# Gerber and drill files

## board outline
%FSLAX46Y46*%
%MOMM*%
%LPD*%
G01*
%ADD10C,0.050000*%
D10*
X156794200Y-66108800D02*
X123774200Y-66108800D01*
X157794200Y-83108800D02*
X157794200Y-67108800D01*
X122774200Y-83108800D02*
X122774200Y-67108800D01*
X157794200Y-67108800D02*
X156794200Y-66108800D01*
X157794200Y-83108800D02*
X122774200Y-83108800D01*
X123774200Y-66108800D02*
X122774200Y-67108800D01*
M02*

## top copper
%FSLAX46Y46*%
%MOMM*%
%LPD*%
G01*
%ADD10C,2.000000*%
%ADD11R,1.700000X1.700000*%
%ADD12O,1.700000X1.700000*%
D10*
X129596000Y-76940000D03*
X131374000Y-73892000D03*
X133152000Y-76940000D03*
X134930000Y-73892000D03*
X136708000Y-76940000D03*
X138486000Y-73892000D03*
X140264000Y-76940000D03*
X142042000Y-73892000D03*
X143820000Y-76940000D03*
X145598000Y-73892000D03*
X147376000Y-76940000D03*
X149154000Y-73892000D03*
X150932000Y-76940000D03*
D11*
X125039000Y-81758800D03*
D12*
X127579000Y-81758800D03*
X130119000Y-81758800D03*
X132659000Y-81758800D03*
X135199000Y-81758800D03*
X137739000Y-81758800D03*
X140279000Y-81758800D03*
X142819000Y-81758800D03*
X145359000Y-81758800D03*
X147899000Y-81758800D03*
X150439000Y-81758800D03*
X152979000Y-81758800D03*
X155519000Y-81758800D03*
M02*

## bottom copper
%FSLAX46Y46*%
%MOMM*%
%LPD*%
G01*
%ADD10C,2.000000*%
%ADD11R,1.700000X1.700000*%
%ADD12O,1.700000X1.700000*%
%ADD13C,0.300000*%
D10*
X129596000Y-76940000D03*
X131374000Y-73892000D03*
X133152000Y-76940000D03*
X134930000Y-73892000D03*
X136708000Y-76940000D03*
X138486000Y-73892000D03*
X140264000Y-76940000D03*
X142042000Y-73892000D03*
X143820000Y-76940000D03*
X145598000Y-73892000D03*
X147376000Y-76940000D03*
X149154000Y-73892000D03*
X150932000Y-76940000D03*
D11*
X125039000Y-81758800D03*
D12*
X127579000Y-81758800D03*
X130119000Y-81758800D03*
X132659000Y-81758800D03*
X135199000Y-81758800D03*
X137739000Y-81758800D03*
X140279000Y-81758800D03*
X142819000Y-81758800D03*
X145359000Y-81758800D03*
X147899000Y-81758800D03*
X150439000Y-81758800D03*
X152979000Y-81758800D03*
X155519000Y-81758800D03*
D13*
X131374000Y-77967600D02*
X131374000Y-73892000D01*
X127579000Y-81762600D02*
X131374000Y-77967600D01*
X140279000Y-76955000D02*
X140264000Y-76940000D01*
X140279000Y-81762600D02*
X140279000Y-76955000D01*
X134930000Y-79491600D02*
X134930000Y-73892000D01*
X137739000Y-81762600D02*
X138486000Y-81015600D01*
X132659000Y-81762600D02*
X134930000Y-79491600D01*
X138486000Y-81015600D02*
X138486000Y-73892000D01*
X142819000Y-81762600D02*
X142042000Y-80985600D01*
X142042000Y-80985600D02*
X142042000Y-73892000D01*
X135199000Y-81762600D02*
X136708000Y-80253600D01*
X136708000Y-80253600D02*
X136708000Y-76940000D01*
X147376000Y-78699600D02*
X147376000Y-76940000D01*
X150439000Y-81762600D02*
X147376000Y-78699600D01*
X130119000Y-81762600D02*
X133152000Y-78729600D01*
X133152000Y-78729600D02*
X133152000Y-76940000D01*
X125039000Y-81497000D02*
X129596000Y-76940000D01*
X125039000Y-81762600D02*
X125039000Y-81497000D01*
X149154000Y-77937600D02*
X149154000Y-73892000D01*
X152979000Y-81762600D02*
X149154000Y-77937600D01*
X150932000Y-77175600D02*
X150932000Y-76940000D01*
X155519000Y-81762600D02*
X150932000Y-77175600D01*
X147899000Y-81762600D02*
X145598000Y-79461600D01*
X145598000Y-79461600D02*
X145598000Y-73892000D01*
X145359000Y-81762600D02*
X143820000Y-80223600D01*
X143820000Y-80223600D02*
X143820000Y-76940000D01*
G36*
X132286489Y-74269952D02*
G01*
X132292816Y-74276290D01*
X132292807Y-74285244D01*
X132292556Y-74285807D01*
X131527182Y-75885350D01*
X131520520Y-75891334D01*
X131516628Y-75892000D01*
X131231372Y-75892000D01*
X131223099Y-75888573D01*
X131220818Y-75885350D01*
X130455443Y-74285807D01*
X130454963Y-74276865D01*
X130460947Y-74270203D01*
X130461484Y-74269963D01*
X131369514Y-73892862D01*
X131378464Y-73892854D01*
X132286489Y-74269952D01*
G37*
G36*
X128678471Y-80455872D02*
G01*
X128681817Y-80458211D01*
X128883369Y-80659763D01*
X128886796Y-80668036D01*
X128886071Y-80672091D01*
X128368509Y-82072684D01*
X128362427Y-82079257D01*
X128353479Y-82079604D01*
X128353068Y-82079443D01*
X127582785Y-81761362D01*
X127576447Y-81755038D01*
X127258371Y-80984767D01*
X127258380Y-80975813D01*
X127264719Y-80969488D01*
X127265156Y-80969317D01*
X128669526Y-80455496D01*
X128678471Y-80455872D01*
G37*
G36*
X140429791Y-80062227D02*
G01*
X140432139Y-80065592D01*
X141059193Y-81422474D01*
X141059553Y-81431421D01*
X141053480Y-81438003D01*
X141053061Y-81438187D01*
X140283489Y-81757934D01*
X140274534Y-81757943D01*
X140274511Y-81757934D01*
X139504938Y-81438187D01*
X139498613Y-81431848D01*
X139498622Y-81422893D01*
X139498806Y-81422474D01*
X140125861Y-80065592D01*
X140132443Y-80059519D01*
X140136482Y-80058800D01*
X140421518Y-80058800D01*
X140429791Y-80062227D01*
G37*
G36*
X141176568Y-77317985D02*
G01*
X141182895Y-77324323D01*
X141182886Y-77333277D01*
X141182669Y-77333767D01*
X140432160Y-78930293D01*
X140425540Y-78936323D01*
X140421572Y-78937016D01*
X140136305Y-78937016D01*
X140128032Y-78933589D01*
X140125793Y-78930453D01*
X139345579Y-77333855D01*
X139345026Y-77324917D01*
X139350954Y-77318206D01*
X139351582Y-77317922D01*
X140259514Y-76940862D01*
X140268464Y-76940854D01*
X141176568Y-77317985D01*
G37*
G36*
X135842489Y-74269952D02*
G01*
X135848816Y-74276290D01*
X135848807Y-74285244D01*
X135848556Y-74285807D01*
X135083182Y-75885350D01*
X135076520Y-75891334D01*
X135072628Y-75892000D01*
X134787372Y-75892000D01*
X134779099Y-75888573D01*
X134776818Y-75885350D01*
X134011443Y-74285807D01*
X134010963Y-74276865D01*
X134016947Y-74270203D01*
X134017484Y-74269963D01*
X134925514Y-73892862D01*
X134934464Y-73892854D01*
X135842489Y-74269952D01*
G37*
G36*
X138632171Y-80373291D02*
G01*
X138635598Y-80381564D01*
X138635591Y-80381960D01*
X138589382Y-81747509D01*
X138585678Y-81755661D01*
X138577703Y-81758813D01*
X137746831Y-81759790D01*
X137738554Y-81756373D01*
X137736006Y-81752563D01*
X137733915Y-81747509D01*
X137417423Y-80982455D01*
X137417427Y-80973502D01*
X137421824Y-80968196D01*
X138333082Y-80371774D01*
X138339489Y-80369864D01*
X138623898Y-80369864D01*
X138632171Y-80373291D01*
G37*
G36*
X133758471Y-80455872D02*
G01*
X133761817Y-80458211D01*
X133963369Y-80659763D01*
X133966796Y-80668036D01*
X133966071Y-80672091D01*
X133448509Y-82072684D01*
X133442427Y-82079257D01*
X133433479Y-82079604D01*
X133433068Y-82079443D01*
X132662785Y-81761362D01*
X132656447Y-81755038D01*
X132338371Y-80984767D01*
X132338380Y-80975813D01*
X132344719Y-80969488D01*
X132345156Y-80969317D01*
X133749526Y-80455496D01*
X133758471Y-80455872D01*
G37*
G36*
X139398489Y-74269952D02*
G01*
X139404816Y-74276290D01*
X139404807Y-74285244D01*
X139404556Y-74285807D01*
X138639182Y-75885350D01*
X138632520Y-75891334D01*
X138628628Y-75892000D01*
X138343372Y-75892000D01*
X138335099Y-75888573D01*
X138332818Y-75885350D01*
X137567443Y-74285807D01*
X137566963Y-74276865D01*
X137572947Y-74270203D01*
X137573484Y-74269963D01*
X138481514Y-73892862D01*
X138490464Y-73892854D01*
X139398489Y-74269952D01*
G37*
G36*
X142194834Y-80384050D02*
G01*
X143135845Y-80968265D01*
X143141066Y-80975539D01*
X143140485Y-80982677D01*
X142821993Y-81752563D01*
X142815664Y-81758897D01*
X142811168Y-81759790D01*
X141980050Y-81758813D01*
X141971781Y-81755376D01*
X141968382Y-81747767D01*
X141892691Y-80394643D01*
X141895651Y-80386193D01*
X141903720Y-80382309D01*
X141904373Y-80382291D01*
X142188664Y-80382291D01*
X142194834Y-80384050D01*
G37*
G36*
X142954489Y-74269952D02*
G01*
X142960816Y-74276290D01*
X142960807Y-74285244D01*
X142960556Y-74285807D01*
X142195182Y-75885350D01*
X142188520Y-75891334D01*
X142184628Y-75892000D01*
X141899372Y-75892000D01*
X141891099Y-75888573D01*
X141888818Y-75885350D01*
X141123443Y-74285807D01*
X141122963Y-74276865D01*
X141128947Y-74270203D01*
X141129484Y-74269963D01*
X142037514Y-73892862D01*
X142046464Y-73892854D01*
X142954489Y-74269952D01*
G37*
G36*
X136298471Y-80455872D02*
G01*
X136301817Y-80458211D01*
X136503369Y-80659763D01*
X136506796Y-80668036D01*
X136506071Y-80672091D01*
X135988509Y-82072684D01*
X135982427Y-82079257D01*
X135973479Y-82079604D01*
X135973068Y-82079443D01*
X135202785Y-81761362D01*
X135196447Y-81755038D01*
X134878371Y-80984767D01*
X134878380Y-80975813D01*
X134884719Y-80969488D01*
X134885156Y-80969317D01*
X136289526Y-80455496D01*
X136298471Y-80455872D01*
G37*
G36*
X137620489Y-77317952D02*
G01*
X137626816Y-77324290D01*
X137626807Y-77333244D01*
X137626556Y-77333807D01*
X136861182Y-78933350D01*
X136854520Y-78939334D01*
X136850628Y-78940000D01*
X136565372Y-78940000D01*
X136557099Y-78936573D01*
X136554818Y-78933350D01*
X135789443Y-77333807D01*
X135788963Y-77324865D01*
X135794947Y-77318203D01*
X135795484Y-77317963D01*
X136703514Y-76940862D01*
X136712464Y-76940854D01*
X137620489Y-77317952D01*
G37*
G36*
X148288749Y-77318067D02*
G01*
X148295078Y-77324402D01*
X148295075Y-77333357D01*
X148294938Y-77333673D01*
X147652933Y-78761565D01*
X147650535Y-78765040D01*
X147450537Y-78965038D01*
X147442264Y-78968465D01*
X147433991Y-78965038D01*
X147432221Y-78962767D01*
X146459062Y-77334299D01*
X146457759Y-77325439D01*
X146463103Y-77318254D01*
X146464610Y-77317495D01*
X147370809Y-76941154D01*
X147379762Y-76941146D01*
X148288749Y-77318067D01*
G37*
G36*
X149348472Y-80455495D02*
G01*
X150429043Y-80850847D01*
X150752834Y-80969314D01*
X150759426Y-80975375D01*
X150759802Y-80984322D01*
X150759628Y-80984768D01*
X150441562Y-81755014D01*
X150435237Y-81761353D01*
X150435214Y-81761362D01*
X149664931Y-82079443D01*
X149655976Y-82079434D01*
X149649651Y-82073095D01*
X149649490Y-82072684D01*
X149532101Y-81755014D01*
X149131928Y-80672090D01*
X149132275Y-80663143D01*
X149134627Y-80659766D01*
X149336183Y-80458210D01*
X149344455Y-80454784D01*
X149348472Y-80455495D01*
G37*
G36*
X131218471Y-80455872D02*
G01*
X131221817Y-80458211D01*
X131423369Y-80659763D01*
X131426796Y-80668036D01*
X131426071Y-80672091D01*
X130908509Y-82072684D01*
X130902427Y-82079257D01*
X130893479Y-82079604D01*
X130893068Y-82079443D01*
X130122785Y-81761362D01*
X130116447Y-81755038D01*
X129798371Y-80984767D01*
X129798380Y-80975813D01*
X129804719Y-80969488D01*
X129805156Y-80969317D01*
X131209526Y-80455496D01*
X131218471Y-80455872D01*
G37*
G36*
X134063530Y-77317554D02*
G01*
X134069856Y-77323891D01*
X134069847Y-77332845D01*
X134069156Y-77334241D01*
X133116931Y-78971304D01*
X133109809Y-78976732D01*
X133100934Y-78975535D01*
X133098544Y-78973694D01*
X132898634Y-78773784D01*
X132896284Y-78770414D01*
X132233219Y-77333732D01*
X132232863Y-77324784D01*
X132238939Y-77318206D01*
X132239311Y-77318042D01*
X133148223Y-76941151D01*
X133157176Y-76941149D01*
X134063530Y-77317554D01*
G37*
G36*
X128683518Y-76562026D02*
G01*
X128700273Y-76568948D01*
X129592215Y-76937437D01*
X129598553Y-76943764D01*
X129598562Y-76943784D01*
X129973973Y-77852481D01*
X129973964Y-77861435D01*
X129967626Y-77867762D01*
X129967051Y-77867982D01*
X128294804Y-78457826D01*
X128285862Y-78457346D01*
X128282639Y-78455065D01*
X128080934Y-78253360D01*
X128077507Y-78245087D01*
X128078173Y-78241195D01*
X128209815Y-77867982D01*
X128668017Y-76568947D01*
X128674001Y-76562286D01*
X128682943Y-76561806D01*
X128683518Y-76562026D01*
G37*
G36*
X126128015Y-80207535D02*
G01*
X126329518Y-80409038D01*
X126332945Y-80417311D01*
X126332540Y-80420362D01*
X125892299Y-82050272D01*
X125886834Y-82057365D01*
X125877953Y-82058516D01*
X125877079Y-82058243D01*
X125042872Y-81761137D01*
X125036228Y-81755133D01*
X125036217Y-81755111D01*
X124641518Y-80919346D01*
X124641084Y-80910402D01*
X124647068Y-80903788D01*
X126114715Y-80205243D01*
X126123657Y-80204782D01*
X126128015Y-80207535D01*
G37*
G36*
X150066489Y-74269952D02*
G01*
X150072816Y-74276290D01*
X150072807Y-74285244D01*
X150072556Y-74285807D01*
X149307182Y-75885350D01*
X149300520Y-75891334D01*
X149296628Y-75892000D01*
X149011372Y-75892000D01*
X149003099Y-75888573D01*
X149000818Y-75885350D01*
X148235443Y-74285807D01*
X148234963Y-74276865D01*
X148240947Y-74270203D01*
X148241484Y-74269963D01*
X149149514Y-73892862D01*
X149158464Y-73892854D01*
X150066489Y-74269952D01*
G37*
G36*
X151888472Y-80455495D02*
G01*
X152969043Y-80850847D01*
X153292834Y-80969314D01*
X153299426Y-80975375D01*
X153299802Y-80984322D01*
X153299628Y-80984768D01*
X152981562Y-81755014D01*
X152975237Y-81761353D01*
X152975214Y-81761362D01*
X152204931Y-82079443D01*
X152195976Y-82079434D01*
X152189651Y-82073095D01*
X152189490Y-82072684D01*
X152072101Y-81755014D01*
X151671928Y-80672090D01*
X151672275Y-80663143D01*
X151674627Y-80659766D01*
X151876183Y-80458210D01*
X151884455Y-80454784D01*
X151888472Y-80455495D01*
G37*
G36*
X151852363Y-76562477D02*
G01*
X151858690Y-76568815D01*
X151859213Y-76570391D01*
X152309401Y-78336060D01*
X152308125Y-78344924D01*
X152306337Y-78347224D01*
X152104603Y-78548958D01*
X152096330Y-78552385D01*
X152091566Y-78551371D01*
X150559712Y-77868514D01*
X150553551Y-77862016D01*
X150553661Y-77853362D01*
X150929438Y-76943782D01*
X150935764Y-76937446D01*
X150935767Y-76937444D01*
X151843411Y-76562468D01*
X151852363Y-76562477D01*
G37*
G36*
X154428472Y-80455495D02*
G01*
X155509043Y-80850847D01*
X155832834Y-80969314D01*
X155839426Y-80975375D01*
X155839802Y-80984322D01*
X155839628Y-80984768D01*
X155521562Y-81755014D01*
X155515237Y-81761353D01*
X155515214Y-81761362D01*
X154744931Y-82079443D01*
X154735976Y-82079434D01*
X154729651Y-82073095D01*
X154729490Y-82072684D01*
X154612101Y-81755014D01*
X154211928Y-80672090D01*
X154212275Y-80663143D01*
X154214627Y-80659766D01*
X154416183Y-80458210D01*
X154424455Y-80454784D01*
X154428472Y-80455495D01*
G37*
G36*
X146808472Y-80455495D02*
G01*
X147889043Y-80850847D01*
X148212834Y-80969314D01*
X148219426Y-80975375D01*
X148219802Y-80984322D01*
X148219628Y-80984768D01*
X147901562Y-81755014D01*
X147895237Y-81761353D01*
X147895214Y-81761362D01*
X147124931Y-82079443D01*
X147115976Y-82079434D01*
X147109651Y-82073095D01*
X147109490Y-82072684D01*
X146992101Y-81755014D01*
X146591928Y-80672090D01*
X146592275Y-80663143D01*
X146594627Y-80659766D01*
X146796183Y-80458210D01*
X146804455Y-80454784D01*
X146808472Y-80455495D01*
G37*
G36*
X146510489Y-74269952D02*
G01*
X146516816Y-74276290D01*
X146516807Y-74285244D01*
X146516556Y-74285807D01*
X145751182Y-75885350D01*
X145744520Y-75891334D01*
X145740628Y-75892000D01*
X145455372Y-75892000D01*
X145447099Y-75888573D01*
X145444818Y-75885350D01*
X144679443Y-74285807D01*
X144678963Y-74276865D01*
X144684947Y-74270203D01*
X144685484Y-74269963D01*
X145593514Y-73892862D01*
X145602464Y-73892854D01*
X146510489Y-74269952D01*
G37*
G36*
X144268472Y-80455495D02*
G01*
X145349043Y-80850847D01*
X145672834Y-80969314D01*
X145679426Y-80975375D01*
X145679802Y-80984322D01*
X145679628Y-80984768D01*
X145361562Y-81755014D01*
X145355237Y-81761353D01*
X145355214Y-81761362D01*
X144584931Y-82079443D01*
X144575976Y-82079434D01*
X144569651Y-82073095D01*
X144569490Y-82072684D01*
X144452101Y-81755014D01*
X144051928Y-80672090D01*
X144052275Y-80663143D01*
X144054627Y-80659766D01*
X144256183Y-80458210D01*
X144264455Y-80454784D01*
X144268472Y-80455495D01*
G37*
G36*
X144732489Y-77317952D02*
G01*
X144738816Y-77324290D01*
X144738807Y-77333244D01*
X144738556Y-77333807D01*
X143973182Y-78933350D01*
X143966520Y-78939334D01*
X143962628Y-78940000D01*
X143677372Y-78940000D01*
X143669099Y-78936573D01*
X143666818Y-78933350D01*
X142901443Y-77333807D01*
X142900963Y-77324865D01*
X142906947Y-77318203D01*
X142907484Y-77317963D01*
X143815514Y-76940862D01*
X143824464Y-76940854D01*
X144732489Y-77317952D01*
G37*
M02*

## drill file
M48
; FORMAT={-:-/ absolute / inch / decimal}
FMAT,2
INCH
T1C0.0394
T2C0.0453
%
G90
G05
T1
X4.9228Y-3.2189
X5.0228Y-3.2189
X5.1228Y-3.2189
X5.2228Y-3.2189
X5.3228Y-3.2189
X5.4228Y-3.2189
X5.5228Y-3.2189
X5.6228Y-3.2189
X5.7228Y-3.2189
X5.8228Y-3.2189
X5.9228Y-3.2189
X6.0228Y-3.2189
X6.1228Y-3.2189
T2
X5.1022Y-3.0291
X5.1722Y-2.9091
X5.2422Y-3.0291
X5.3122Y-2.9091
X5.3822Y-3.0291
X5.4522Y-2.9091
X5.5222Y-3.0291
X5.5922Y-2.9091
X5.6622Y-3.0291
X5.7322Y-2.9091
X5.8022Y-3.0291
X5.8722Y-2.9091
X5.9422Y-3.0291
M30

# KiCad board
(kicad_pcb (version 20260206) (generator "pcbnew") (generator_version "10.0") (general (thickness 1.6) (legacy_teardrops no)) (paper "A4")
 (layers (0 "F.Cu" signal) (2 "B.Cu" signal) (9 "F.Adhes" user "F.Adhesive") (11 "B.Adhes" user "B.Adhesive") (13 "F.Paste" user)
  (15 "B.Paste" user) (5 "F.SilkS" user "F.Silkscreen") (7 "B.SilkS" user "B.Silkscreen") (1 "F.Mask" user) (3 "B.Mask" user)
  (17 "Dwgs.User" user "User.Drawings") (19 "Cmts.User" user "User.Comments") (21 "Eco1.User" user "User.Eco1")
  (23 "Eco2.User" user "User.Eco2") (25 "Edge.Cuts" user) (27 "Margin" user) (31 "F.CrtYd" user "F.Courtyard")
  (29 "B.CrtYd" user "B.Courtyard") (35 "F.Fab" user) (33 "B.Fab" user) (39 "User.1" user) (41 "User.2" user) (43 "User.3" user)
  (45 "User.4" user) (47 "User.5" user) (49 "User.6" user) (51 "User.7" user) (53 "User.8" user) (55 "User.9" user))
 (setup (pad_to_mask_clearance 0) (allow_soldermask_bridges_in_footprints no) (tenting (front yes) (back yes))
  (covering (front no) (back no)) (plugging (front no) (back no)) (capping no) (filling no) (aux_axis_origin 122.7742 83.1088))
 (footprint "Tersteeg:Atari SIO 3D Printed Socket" (layer "F.Cu") (at 129.596 83.036)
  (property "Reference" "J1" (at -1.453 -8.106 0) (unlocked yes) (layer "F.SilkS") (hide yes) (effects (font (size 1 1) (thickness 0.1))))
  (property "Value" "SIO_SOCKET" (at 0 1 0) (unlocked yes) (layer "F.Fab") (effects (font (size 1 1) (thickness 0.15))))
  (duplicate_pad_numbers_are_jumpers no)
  (pad "1" thru_hole circle (at 0 -6.096) (size 2 2) (drill 1.15) (layers "*.Cu" "*.Mask") (remove_unused_layers no)
   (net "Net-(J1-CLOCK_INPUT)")
   (teardrops (best_length_ratio 0.5) (max_length 1) (best_width_ratio 1) (max_width 2) (curved_edges no) (filter_ratio 0.9) (enabled yes)
    (allow_two_segments yes) (prefer_zone_connections yes)))
  (pad "2" thru_hole circle (at 1.778 -9.144) (size 2 2) (drill 1.15) (layers "*.Cu" "*.Mask") (remove_unused_layers no)
   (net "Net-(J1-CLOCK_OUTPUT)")
   (teardrops (best_length_ratio 0.5) (max_length 1) (best_width_ratio 1) (max_width 2) (curved_edges no) (filter_ratio 0.9) (enabled yes)
    (allow_two_segments yes) (prefer_zone_connections yes)))
  (pad "3" thru_hole circle (at 3.556 -6.096) (size 2 2) (drill 1.15) (layers "*.Cu" "*.Mask") (remove_unused_layers no)
   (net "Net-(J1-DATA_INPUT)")
   (teardrops (best_length_ratio 0.5) (max_length 1) (best_width_ratio 1) (max_width 2) (curved_edges no) (filter_ratio 0.9) (enabled yes)
    (allow_two_segments yes) (prefer_zone_connections yes)))
  (pad "4" thru_hole circle (at 5.334 -9.144) (size 2 2) (drill 1.15) (layers "*.Cu" "*.Mask") (remove_unused_layers no) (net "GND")
   (teardrops (best_length_ratio 0.5) (max_length 1) (best_width_ratio 1) (max_width 2) (curved_edges no) (filter_ratio 0.9) (enabled yes)
    (allow_two_segments yes) (prefer_zone_connections yes)))
  (pad "5" thru_hole circle (at 7.112 -6.096) (size 2 2) (drill 1.15) (layers "*.Cu" "*.Mask") (remove_unused_layers no)
   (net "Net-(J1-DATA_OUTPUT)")
   (teardrops (best_length_ratio 0.5) (max_length 1) (best_width_ratio 1) (max_width 2) (curved_edges no) (filter_ratio 0.9) (enabled yes)
    (allow_two_segments yes) (prefer_zone_connections yes)))
  (pad "6" thru_hole circle (at 8.89 -9.144) (size 2 2) (drill 1.15) (layers "*.Cu" "*.Mask") (remove_unused_layers no) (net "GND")
   (teardrops (best_length_ratio 0.5) (max_length 1) (best_width_ratio 1) (max_width 2) (curved_edges no) (filter_ratio 0.9) (enabled yes)
    (allow_two_segments yes) (prefer_zone_connections yes)))
  (pad "7" thru_hole circle (at 10.668 -6.096) (size 2 2) (drill 1.15) (layers "*.Cu" "*.Mask") (remove_unused_layers no)
   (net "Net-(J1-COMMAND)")
   (teardrops (best_length_ratio 0.5) (max_length 1) (best_width_ratio 1) (max_width 2) (curved_edges no) (filter_ratio 0.9) (enabled yes)
    (allow_two_segments yes) (prefer_zone_connections yes)))
  (pad "8" thru_hole circle (at 12.446 -9.144) (size 2 2) (drill 1.15) (layers "*.Cu" "*.Mask") (remove_unused_layers no)
   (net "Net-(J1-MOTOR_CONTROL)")
   (teardrops (best_length_ratio 0.5) (max_length 1) (best_width_ratio 1) (max_width 2) (curved_edges no) (filter_ratio 0.9) (enabled yes)
    (allow_two_segments yes) (prefer_zone_connections yes)))
  (pad "9" thru_hole circle (at 14.224 -6.096) (size 2 2) (drill 1.15) (layers "*.Cu" "*.Mask") (remove_unused_layers no)
   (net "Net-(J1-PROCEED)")
   (teardrops (best_length_ratio 0.5) (max_length 1) (best_width_ratio 1) (max_width 2) (curved_edges no) (filter_ratio 0.9) (enabled yes)
    (allow_two_segments yes) (prefer_zone_connections yes)))
  (pad "10" thru_hole circle (at 16.002 -9.144) (size 2 2) (drill 1.15) (layers "*.Cu" "*.Mask") (remove_unused_layers no) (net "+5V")
   (teardrops (best_length_ratio 0.5) (max_length 1) (best_width_ratio 1) (max_width 2) (curved_edges no) (filter_ratio 0.9) (enabled yes)
    (allow_two_segments yes) (prefer_zone_connections yes)))
  (pad "11" thru_hole circle (at 17.78 -6.096) (size 2 2) (drill 1.15) (layers "*.Cu" "*.Mask") (remove_unused_layers no)
   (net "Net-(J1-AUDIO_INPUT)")
   (teardrops (best_length_ratio 0.5) (max_length 1) (best_width_ratio 1) (max_width 2) (curved_edges no) (filter_ratio 0.9) (enabled yes)
    (allow_two_segments yes) (prefer_zone_connections yes)))
  (pad "12" thru_hole circle (at 19.558 -9.144) (size 2 2) (drill 1.15) (layers "*.Cu" "*.Mask") (remove_unused_layers no) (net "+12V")
   (teardrops (best_length_ratio 0.5) (max_length 1) (best_width_ratio 1) (max_width 2) (curved_edges no) (filter_ratio 0.9) (enabled yes)
    (allow_two_segments yes) (prefer_zone_connections yes)))
  (pad "13" thru_hole circle (at 21.336 -6.096) (size 2 2) (drill 1.15) (layers "*.Cu" "*.Mask") (remove_unused_layers no)
   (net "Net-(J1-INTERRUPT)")
   (teardrops (best_length_ratio 0.5) (max_length 1) (best_width_ratio 1) (max_width 2) (curved_edges no) (filter_ratio 0.9) (enabled yes)
    (allow_two_segments yes) (prefer_zone_connections yes))))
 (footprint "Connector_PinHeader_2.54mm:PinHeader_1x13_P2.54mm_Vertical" (layer "B.Cu") (at 125.039 81.7588 -90)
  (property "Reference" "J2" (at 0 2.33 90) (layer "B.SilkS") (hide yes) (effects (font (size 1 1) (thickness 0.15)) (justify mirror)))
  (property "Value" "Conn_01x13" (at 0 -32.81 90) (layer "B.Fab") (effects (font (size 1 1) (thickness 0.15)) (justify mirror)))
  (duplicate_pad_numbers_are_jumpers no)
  (pad "1" thru_hole rect (at 0 0 270) (size 1.7 1.7) (drill 1) (layers "*.Cu" "*.Mask") (remove_unused_layers no)
   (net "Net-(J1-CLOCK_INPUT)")
   (teardrops (best_length_ratio 0.5) (max_length 1) (best_width_ratio 1) (max_width 2) (curved_edges no) (filter_ratio 0.9) (enabled yes)
    (allow_two_segments yes) (prefer_zone_connections yes)))
  (pad "2" thru_hole oval (at 0 -2.54 270) (size 1.7 1.7) (drill 1) (layers "*.Cu" "*.Mask") (remove_unused_layers no)
   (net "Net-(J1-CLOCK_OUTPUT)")
   (teardrops (best_length_ratio 0.5) (max_length 1) (best_width_ratio 1) (max_width 2) (curved_edges no) (filter_ratio 0.9) (enabled yes)
    (allow_two_segments yes) (prefer_zone_connections yes)))
  (pad "3" thru_hole oval (at 0 -5.08 270) (size 1.7 1.7) (drill 1) (layers "*.Cu" "*.Mask") (remove_unused_layers no)
   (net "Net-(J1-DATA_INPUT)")
   (teardrops (best_length_ratio 0.5) (max_length 1) (best_width_ratio 1) (max_width 2) (curved_edges no) (filter_ratio 0.9) (enabled yes)
    (allow_two_segments yes) (prefer_zone_connections yes)))
  (pad "4" thru_hole oval (at 0 -7.62 270) (size 1.7 1.7) (drill 1) (layers "*.Cu" "*.Mask") (remove_unused_layers no) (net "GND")
   (teardrops (best_length_ratio 0.5) (max_length 1) (best_width_ratio 1) (max_width 2) (curved_edges no) (filter_ratio 0.9) (enabled yes)
    (allow_two_segments yes) (prefer_zone_connections yes)))
  (pad "5" thru_hole oval (at 0 -10.16 270) (size 1.7 1.7) (drill 1) (layers "*.Cu" "*.Mask") (remove_unused_layers no)
   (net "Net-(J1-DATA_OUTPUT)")
   (teardrops (best_length_ratio 0.5) (max_length 1) (best_width_ratio 1) (max_width 2) (curved_edges no) (filter_ratio 0.9) (enabled yes)
    (allow_two_segments yes) (prefer_zone_connections yes)))
  (pad "6" thru_hole oval (at 0 -12.7 270) (size 1.7 1.7) (drill 1) (layers "*.Cu" "*.Mask") (remove_unused_layers no) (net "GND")
   (teardrops (best_length_ratio 0.5) (max_length 1) (best_width_ratio 1) (max_width 2) (curved_edges no) (filter_ratio 0.9) (enabled yes)
    (allow_two_segments yes) (prefer_zone_connections yes)))
  (pad "7" thru_hole oval (at 0 -15.24 270) (size 1.7 1.7) (drill 1) (layers "*.Cu" "*.Mask") (remove_unused_layers no)
   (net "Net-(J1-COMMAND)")
   (teardrops (best_length_ratio 0.5) (max_length 1) (best_width_ratio 1) (max_width 2) (curved_edges no) (filter_ratio 0.9) (enabled yes)
    (allow_two_segments yes) (prefer_zone_connections yes)))
  (pad "8" thru_hole oval (at 0 -17.78 270) (size 1.7 1.7) (drill 1) (layers "*.Cu" "*.Mask") (remove_unused_layers no)
   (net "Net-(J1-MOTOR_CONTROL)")
   (teardrops (best_length_ratio 0.5) (max_length 1) (best_width_ratio 1) (max_width 2) (curved_edges no) (filter_ratio 0.9) (enabled yes)
    (allow_two_segments yes) (prefer_zone_connections yes)))
  (pad "9" thru_hole oval (at 0 -20.32 270) (size 1.7 1.7) (drill 1) (layers "*.Cu" "*.Mask") (remove_unused_layers no)
   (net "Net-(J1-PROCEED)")
   (teardrops (best_length_ratio 0.5) (max_length 1) (best_width_ratio 1) (max_width 2) (curved_edges no) (filter_ratio 0.9) (enabled yes)
    (allow_two_segments yes) (prefer_zone_connections yes)))
  (pad "10" thru_hole oval (at 0 -22.86 270) (size 1.7 1.7) (drill 1) (layers "*.Cu" "*.Mask") (remove_unused_layers no) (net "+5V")
   (teardrops (best_length_ratio 0.5) (max_length 1) (best_width_ratio 1) (max_width 2) (curved_edges no) (filter_ratio 0.9) (enabled yes)
    (allow_two_segments yes) (prefer_zone_connections yes)))
  (pad "11" thru_hole oval (at 0 -25.4 270) (size 1.7 1.7) (drill 1) (layers "*.Cu" "*.Mask") (remove_unused_layers no)
   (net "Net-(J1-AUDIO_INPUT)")
   (teardrops (best_length_ratio 0.5) (max_length 1) (best_width_ratio 1) (max_width 2) (curved_edges no) (filter_ratio 0.9) (enabled yes)
    (allow_two_segments yes) (prefer_zone_connections yes)))
  (pad "12" thru_hole oval (at 0 -27.94 270) (size 1.7 1.7) (drill 1) (layers "*.Cu" "*.Mask") (remove_unused_layers no) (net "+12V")
   (teardrops (best_length_ratio 0.5) (max_length 1) (best_width_ratio 1) (max_width 2) (curved_edges no) (filter_ratio 0.9) (enabled yes)
    (allow_two_segments yes) (prefer_zone_connections yes)))
  (pad "13" thru_hole oval (at 0 -30.48 270) (size 1.7 1.7) (drill 1) (layers "*.Cu" "*.Mask") (remove_unused_layers no)
   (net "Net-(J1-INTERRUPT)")
   (teardrops (best_length_ratio 0.5) (max_length 1) (best_width_ratio 1) (max_width 2) (curved_edges no) (filter_ratio 0.9) (enabled yes)
    (allow_two_segments yes) (prefer_zone_connections yes))))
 (gr_line (start 122.7742 83.1088) (end 122.7742 67.1088) (stroke (width 0.05) (type default)) (layer "Edge.Cuts"))
 (gr_line (start 123.7742 66.1088) (end 122.7742 67.1088) (stroke (width 0.05) (type default)) (layer "Edge.Cuts"))
 (gr_line (start 156.7942 66.1088) (end 123.7742 66.1088) (stroke (width 0.05) (type default)) (layer "Edge.Cuts"))
 (gr_line (start 157.7942 67.1088) (end 156.7942 66.1088) (stroke (width 0.05) (type default)) (layer "Edge.Cuts"))
 (gr_line (start 157.7942 83.1088) (end 122.7742 83.1088) (stroke (width 0.05) (type default)) (layer "Edge.Cuts"))
 (gr_line (start 157.7942 83.1088) (end 157.7942 67.1088) (stroke (width 0.05) (type default)) (layer "Edge.Cuts"))
 (segment (start 131.374 77.9676) (end 131.374 73.892) (width 0.3) (layer "B.Cu") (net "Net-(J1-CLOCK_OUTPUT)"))
 (segment (start 127.579 81.7626) (end 131.374 77.9676) (width 0.3) (layer "B.Cu") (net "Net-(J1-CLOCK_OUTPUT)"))
 (segment (start 140.279 76.955) (end 140.264 76.94) (width 0.3) (layer "B.Cu") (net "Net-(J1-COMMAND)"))
 (segment (start 140.279 81.7626) (end 140.279 76.955) (width 0.3) (layer "B.Cu") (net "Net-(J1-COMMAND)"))
 (segment (start 134.93 79.4916) (end 134.93 73.892) (width 0.3) (layer "B.Cu") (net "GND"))
 (segment (start 137.739 81.7626) (end 138.486 81.0156) (width 0.3) (layer "B.Cu") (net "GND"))
 (segment (start 132.659 81.7626) (end 134.93 79.4916) (width 0.3) (layer "B.Cu") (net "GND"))
 (segment (start 138.486 81.0156) (end 138.486 73.892) (width 0.3) (layer "B.Cu") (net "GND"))
 (segment (start 142.819 81.7626) (end 142.042 80.9856) (width 0.3) (layer "B.Cu") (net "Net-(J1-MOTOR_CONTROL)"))
 (segment (start 142.042 80.9856) (end 142.042 73.892) (width 0.3) (layer "B.Cu") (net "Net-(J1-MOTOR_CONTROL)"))
 (segment (start 135.199 81.7626) (end 136.708 80.2536) (width 0.3) (layer "B.Cu") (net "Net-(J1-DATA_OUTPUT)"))
 (segment (start 136.708 80.2536) (end 136.708 76.94) (width 0.3) (layer "B.Cu") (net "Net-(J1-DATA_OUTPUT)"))
 (segment (start 147.376 78.6996) (end 147.376 76.94) (width 0.3) (layer "B.Cu") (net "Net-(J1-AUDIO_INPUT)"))
 (segment (start 150.439 81.7626) (end 147.376 78.6996) (width 0.3) (layer "B.Cu") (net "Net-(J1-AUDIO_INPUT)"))
 (segment (start 130.119 81.7626) (end 133.152 78.7296) (width 0.3) (layer "B.Cu") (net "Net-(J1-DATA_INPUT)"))
 (segment (start 133.152 78.7296) (end 133.152 76.94) (width 0.3) (layer "B.Cu") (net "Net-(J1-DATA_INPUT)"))
 (segment (start 125.039 81.497) (end 129.596 76.94) (width 0.3) (layer "B.Cu") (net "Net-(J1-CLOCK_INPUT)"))
 (segment (start 125.039 81.7626) (end 125.039 81.497) (width 0.3) (layer "B.Cu") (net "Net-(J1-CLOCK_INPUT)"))
 (segment (start 149.154 77.9376) (end 149.154 73.892) (width 0.3) (layer "B.Cu") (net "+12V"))
 (segment (start 152.979 81.7626) (end 149.154 77.9376) (width 0.3) (layer "B.Cu") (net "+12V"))
 (segment (start 150.932 77.1756) (end 150.932 76.94) (width 0.3) (layer "B.Cu") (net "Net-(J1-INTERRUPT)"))
 (segment (start 155.519 81.7626) (end 150.932 77.1756) (width 0.3) (layer "B.Cu") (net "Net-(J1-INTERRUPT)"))
 (segment (start 147.899 81.7626) (end 145.598 79.4616) (width 0.3) (layer "B.Cu") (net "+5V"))
 (segment (start 145.598 79.4616) (end 145.598 73.892) (width 0.3) (layer "B.Cu") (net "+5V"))
 (segment (start 145.359 81.7626) (end 143.82 80.2236) (width 0.3) (layer "B.Cu") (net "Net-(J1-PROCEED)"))
 (segment (start 143.82 80.2236) (end 143.82 76.94) (width 0.3) (layer "B.Cu") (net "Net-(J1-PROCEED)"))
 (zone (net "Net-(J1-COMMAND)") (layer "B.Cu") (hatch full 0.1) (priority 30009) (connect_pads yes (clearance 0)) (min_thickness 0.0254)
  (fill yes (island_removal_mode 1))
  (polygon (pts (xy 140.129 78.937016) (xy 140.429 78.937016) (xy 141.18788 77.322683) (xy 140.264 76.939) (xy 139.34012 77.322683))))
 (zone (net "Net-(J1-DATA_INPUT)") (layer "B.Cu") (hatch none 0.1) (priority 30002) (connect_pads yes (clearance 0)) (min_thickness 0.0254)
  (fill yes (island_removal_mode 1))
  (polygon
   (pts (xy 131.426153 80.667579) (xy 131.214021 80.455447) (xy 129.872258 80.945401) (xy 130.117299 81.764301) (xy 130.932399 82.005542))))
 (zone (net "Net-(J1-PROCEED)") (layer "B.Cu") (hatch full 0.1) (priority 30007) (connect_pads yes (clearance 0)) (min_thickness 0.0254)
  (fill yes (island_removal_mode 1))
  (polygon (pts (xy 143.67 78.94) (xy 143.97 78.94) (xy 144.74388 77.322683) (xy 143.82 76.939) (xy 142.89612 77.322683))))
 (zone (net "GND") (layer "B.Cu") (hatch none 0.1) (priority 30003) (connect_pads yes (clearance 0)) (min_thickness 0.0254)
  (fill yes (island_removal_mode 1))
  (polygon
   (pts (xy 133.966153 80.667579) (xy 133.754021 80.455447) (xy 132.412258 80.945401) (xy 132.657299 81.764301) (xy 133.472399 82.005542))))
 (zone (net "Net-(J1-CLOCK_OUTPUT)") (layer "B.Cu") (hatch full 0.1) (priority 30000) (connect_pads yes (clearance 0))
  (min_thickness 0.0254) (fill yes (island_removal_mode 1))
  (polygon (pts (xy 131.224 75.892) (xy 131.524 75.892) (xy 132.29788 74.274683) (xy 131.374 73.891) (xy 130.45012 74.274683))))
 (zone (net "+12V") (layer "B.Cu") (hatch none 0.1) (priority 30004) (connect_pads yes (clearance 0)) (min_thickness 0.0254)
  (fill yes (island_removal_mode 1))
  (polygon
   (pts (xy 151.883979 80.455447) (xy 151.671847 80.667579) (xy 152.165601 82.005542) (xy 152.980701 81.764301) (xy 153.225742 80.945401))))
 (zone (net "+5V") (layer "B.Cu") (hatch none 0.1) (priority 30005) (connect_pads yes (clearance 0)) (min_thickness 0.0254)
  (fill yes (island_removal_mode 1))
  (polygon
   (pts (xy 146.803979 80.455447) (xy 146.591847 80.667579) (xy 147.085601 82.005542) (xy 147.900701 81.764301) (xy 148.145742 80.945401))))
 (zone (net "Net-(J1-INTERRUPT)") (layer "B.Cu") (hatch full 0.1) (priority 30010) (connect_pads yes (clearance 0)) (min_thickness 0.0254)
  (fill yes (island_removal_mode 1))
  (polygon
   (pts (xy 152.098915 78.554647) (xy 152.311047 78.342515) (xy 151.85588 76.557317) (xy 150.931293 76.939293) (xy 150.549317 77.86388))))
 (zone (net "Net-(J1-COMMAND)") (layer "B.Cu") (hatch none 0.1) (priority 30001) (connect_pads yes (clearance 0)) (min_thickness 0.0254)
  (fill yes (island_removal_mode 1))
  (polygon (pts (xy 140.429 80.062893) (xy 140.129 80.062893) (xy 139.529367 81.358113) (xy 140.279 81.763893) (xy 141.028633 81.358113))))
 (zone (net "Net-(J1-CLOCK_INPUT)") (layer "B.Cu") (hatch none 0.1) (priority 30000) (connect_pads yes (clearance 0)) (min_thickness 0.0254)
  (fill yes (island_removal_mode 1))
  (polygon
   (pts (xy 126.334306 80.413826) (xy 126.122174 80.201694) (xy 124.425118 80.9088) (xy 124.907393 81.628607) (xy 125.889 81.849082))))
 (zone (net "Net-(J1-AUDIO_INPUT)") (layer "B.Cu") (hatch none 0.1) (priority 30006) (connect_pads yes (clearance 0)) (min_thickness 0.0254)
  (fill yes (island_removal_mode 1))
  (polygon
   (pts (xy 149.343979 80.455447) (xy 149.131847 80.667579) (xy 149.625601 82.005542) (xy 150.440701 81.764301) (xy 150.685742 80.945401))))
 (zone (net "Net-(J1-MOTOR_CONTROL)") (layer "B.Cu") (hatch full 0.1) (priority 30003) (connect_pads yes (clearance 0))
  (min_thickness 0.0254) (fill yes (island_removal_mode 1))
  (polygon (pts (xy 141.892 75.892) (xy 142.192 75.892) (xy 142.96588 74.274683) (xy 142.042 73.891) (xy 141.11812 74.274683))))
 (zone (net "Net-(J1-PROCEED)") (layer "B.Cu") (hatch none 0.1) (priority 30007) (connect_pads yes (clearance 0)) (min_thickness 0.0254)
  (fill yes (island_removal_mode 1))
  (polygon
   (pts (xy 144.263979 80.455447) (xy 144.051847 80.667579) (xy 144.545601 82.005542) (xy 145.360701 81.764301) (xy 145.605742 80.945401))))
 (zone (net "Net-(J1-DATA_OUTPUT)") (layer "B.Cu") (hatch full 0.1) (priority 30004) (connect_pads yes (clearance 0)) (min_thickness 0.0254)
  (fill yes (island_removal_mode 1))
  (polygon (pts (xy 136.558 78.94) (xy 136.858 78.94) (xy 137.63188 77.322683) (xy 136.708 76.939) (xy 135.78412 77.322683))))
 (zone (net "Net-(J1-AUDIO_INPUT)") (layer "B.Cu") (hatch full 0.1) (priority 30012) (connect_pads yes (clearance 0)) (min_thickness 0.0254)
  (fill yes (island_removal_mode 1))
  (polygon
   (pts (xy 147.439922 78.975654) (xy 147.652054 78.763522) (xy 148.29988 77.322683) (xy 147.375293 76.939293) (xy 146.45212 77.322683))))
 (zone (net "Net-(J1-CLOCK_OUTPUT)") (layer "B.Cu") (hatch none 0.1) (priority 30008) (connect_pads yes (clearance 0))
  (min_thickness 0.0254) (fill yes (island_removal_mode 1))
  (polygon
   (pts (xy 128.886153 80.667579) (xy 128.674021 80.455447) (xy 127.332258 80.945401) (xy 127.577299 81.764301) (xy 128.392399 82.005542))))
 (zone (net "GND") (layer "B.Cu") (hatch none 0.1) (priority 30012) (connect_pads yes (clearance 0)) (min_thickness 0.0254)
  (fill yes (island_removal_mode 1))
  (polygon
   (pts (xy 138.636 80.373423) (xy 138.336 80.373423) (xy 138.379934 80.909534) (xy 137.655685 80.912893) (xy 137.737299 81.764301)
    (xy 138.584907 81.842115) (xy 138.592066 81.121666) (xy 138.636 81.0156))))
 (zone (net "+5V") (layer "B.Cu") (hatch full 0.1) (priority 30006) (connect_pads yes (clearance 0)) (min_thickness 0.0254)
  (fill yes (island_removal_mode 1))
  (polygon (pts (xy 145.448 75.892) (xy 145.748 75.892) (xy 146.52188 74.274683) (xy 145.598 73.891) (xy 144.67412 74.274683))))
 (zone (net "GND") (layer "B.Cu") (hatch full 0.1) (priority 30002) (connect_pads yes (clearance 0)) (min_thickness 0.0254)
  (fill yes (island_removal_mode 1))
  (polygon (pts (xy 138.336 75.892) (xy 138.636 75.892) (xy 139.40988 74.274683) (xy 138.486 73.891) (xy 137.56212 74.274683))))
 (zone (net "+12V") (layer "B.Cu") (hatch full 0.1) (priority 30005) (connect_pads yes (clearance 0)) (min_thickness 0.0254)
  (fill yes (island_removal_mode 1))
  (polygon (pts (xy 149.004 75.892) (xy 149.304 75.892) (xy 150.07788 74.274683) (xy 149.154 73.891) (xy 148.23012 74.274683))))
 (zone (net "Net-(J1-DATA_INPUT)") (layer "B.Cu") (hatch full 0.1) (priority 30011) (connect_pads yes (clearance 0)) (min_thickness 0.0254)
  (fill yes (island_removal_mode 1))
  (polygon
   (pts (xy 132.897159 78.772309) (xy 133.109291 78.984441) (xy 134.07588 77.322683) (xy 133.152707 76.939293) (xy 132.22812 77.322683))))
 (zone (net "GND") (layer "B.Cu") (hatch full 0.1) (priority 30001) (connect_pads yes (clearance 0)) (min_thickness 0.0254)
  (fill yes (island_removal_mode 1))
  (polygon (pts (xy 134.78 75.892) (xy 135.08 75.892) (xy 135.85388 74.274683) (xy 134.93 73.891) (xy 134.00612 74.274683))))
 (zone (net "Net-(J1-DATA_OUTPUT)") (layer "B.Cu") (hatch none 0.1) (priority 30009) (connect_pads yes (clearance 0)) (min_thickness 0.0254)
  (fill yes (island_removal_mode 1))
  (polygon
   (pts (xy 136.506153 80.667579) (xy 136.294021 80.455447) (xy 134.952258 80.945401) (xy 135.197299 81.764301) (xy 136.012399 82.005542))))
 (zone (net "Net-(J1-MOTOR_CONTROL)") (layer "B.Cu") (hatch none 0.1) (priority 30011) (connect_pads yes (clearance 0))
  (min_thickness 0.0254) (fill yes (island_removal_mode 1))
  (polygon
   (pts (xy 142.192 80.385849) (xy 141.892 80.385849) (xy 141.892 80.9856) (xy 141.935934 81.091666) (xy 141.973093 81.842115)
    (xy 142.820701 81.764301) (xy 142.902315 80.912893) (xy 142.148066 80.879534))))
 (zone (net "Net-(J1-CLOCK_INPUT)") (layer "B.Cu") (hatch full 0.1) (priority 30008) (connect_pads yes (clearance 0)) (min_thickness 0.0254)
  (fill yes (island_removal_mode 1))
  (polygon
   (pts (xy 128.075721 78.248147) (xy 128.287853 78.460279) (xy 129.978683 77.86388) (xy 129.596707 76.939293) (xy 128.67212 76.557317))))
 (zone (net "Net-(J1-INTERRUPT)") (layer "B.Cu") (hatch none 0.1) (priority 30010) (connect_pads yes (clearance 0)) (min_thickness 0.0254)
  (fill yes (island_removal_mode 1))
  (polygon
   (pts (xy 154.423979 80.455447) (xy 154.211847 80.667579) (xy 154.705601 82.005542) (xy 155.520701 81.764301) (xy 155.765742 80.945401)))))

